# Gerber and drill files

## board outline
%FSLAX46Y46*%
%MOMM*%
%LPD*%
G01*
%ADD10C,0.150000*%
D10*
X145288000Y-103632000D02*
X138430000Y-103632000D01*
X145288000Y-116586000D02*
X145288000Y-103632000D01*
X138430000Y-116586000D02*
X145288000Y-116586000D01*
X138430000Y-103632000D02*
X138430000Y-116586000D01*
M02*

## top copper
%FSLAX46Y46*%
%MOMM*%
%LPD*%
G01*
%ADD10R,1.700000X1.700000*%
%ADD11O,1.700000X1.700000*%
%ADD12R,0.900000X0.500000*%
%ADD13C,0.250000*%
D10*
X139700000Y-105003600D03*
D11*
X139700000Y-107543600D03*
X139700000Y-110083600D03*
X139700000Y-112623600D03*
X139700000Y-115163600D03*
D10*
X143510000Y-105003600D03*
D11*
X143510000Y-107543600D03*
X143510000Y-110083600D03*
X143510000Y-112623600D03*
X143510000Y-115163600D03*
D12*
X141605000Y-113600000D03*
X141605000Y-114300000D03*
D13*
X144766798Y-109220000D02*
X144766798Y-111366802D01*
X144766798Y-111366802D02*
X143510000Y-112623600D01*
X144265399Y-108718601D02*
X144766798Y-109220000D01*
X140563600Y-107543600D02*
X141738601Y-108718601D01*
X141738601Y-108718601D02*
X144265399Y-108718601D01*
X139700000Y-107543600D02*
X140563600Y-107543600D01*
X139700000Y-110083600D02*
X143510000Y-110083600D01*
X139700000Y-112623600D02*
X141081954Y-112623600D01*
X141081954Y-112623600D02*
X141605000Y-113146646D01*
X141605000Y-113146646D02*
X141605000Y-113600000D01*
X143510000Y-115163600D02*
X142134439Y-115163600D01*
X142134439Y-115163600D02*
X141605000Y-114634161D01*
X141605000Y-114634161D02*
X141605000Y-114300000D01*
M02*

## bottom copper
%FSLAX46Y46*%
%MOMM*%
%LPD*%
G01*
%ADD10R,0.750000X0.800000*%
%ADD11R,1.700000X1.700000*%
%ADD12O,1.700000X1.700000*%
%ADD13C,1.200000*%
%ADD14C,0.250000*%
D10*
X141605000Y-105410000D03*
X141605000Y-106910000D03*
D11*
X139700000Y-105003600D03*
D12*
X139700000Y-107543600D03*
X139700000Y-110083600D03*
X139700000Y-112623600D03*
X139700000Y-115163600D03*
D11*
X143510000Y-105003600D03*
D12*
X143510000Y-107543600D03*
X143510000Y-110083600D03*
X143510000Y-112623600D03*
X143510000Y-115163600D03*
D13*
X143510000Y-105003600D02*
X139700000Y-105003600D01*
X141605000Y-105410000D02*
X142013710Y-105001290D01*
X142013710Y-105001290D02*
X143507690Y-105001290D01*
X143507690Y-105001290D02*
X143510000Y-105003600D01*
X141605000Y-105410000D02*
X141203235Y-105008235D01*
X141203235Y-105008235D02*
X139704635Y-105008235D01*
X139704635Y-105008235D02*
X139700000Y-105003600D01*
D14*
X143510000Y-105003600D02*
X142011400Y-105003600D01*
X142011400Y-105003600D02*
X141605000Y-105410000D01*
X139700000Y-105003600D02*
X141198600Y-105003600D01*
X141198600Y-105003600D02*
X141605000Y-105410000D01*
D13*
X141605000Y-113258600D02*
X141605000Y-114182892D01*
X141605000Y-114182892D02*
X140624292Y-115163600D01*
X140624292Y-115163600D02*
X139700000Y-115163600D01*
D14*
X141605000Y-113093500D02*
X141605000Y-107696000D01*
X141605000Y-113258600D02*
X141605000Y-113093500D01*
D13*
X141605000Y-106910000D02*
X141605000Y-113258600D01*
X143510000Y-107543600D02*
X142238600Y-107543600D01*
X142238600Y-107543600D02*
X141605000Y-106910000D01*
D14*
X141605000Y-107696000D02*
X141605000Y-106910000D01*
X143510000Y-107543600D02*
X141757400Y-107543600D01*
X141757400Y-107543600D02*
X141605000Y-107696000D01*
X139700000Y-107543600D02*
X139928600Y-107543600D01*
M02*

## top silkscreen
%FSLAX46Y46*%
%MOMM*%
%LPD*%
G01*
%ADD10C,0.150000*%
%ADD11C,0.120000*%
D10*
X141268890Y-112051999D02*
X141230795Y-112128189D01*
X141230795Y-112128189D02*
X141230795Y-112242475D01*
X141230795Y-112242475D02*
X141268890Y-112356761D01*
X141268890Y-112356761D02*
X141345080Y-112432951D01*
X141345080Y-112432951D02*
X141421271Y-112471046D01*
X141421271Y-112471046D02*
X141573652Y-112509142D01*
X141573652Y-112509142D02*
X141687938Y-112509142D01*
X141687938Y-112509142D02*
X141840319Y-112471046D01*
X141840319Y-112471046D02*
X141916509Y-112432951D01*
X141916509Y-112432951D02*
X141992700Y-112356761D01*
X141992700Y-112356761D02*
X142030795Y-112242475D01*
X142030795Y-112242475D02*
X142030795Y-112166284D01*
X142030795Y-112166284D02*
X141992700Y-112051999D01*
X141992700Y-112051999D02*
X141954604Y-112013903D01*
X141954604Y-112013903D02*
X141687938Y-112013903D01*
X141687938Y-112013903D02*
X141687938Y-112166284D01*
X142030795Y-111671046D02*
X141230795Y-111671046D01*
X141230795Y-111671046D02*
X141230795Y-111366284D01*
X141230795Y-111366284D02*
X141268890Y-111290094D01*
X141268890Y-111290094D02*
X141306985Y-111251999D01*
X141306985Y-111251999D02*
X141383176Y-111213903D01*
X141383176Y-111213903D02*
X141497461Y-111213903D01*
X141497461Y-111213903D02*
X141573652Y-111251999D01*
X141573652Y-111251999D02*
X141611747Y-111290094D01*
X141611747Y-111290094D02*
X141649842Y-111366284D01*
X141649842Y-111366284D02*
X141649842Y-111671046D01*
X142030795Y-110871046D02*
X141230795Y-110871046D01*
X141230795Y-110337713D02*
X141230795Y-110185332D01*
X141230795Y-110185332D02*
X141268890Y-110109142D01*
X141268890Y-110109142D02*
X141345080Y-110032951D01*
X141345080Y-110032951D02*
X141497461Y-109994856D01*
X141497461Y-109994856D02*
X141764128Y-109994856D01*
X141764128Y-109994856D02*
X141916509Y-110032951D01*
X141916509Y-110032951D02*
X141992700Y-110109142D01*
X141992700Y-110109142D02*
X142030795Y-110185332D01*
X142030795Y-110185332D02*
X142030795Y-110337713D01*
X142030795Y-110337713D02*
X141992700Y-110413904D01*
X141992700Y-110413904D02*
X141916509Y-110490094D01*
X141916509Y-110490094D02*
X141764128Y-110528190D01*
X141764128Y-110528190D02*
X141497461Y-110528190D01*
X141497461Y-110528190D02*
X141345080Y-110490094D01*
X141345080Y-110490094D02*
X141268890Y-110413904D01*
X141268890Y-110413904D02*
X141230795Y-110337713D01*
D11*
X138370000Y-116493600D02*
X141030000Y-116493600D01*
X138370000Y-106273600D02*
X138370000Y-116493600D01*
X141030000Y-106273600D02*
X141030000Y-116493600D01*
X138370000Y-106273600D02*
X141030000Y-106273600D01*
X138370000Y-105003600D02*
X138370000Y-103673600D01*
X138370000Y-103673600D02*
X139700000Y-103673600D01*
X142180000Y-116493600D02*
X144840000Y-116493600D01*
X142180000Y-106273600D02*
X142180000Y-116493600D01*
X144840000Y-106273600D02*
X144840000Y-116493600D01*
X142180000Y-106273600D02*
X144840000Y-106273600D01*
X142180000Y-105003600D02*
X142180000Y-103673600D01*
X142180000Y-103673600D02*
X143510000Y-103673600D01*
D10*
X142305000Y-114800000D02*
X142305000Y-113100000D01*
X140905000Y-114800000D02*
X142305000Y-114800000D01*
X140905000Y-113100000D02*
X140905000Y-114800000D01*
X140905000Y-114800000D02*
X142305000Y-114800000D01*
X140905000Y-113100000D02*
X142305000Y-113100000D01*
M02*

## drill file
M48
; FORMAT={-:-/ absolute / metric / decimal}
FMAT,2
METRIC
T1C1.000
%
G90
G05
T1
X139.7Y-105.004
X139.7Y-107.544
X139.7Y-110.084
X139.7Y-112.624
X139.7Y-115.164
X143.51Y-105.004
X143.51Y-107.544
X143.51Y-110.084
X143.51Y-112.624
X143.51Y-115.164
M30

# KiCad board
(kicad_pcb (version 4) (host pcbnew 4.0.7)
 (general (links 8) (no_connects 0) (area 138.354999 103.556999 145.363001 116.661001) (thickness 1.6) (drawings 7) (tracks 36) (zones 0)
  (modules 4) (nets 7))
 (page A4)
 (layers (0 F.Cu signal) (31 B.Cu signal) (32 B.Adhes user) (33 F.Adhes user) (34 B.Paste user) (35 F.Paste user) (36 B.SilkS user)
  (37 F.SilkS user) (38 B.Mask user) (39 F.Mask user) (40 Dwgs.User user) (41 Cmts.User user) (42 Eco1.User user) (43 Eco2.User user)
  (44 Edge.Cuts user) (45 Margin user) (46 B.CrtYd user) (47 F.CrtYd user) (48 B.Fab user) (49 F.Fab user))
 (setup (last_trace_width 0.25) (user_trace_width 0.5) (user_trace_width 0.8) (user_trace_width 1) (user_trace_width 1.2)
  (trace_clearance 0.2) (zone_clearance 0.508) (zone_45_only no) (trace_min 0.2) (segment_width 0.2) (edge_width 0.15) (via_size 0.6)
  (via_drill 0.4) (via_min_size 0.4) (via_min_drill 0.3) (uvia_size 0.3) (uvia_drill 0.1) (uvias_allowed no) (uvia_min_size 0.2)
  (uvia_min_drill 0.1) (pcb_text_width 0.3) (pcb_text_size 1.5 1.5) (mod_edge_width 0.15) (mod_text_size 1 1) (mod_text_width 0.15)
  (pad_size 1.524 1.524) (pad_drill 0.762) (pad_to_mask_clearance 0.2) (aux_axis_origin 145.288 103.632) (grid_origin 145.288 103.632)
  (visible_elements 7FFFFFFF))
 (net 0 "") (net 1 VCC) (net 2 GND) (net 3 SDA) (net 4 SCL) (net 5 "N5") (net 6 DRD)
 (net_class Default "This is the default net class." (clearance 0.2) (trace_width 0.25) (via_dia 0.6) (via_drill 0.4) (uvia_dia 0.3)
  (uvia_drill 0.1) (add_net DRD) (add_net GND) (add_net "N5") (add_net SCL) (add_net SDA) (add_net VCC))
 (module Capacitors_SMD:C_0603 (layer B.Cu) (at 141.605 106.16 90)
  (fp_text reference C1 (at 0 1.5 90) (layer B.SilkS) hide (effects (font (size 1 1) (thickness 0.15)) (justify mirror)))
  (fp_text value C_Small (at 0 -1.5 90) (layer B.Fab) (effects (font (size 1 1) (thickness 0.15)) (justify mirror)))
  (pad 2 smd rect (at 0.75 0 90) (size 0.8 0.75) (layers B.Cu B.Paste B.Mask) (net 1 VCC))
  (pad 1 smd rect (at -0.75 0 90) (size 0.8 0.75) (layers B.Cu B.Paste B.Mask) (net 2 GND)))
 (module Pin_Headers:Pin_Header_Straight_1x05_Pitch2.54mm (layer F.Cu) (at 139.7 105.0036)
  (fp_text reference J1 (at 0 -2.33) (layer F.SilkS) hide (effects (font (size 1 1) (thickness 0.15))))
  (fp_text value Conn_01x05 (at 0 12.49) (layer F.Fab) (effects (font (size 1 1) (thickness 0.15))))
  (fp_line (start -1.33 11.49) (end 1.33 11.49) (layer F.SilkS) (width 0.12))
  (fp_line (start -1.33 1.27) (end -1.33 11.49) (layer F.SilkS) (width 0.12))
  (fp_line (start 1.33 1.27) (end 1.33 11.49) (layer F.SilkS) (width 0.12))
  (fp_line (start -1.33 1.27) (end 1.33 1.27) (layer F.SilkS) (width 0.12))
  (fp_line (start -1.33 0) (end -1.33 -1.33) (layer F.SilkS) (width 0.12))
  (fp_line (start -1.33 -1.33) (end 0 -1.33) (layer F.SilkS) (width 0.12))
  (pad 1 thru_hole rect (at 0 0) (size 1.7 1.7) (drill 1) (layers *.Cu *.Mask) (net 1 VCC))
  (pad 2 thru_hole oval (at 0 2.54) (size 1.7 1.7) (drill 1) (layers *.Cu *.Mask) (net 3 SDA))
  (pad 3 thru_hole oval (at 0 5.08) (size 1.7 1.7) (drill 1) (layers *.Cu *.Mask) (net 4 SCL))
  (pad 4 thru_hole oval (at 0 7.62) (size 1.7 1.7) (drill 1) (layers *.Cu *.Mask) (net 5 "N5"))
  (pad 5 thru_hole oval (at 0 10.16) (size 1.7 1.7) (drill 1) (layers *.Cu *.Mask) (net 2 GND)))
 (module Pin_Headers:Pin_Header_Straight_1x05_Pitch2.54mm (layer F.Cu) (at 143.51 105.0036)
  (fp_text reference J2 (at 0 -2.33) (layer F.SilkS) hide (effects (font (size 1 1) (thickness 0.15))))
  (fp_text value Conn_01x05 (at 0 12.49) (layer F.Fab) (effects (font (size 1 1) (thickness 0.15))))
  (fp_line (start -1.33 11.49) (end 1.33 11.49) (layer F.SilkS) (width 0.12))
  (fp_line (start -1.33 1.27) (end -1.33 11.49) (layer F.SilkS) (width 0.12))
  (fp_line (start 1.33 1.27) (end 1.33 11.49) (layer F.SilkS) (width 0.12))
  (fp_line (start -1.33 1.27) (end 1.33 1.27) (layer F.SilkS) (width 0.12))
  (fp_line (start -1.33 0) (end -1.33 -1.33) (layer F.SilkS) (width 0.12))
  (fp_line (start -1.33 -1.33) (end 0 -1.33) (layer F.SilkS) (width 0.12))
  (pad 1 thru_hole rect (at 0 0) (size 1.7 1.7) (drill 1) (layers *.Cu *.Mask) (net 1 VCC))
  (pad 2 thru_hole oval (at 0 2.54) (size 1.7 1.7) (drill 1) (layers *.Cu *.Mask) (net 2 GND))
  (pad 3 thru_hole oval (at 0 5.08) (size 1.7 1.7) (drill 1) (layers *.Cu *.Mask) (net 4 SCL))
  (pad 4 thru_hole oval (at 0 7.62) (size 1.7 1.7) (drill 1) (layers *.Cu *.Mask) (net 3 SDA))
  (pad 5 thru_hole oval (at 0 10.16) (size 1.7 1.7) (drill 1) (layers *.Cu *.Mask) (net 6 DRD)))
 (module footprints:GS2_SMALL (layer F.Cu) (at 141.605 114.3)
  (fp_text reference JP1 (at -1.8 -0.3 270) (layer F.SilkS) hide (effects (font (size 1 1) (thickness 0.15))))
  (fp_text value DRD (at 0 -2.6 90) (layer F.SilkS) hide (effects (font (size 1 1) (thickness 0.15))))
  (fp_line (start 0.7 0.5) (end 0.7 -1.2) (layer F.SilkS) (width 0.15))
  (fp_line (start -0.7 0.5) (end 0.7 0.5) (layer F.SilkS) (width 0.15))
  (fp_line (start -0.7 -1.2) (end -0.7 0.5) (layer F.SilkS) (width 0.15))
  (fp_line (start -0.7 0.5) (end 0.7 0.5) (layer F.SilkS) (width 0.15))
  (fp_line (start -0.7 -1.2) (end 0.7 -1.2) (layer F.SilkS) (width 0.15))
  (pad 1 smd rect (at 0 -0.7) (size 0.9 0.5) (layers F.Cu F.Paste F.Mask) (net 5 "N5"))
  (pad 2 smd rect (at 0 0) (size 0.9 0.5) (layers F.Cu F.Paste F.Mask) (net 6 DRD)))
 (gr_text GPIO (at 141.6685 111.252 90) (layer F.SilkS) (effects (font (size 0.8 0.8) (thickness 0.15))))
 (gr_line (start 145.288 103.632) (end 138.43 103.632) (layer Edge.Cuts) (width 0.15))
 (gr_line (start 145.288 116.586) (end 145.288 103.632) (layer Edge.Cuts) (width 0.15))
 (gr_line (start 138.43 116.586) (end 145.288 116.586) (layer Edge.Cuts) (width 0.15))
 (gr_line (start 138.43 103.632) (end 138.43 116.586) (layer Edge.Cuts) (width 0.15))
 (segment (start 143.51 105.0036) (end 139.7 105.0036) (width 1.2) (layer B.Cu) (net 1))
 (segment (start 141.605 105.41) (end 142.01371 105.00129) (width 1.2) (layer B.Cu) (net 1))
 (segment (start 142.01371 105.00129) (end 143.50769 105.00129) (width 1.2) (layer B.Cu) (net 1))
 (segment (start 143.50769 105.00129) (end 143.51 105.0036) (width 1.2) (layer B.Cu) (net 1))
 (segment (start 141.605 105.41) (end 141.203235 105.008235) (width 1.2) (layer B.Cu) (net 1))
 (segment (start 141.203235 105.008235) (end 139.704635 105.008235) (width 1.2) (layer B.Cu) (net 1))
 (segment (start 139.704635 105.008235) (end 139.7 105.0036) (width 1.2) (layer B.Cu) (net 1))
 (segment (start 143.51 105.0036) (end 142.0114 105.0036) (width 0.25) (layer B.Cu) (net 1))
 (segment (start 142.0114 105.0036) (end 141.605 105.41) (width 0.25) (layer B.Cu) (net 1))
 (segment (start 139.7 105.0036) (end 141.1986 105.0036) (width 0.25) (layer B.Cu) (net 1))
 (segment (start 141.1986 105.0036) (end 141.605 105.41) (width 0.25) (layer B.Cu) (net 1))
 (segment (start 141.605 113.2586) (end 141.605 114.182892) (width 1.2) (layer B.Cu) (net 2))
 (segment (start 141.605 114.182892) (end 140.624292 115.1636) (width 1.2) (layer B.Cu) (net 2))
 (segment (start 140.624292 115.1636) (end 139.7 115.1636) (width 1.2) (layer B.Cu) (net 2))
 (segment (start 141.605 113.0935) (end 141.605 107.696) (width 0.25) (layer B.Cu) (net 2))
 (segment (start 141.605 113.2586) (end 141.605 113.0935) (width 0.25) (layer B.Cu) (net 2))
 (segment (start 141.605 106.91) (end 141.605 113.2586) (width 1.2) (layer B.Cu) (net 2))
 (segment (start 143.51 107.5436) (end 142.2386 107.5436) (width 1.2) (layer B.Cu) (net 2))
 (segment (start 142.2386 107.5436) (end 141.605 106.91) (width 1.2) (layer B.Cu) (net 2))
 (segment (start 141.605 107.696) (end 141.605 106.91) (width 0.25) (layer B.Cu) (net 2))
 (segment (start 143.51 107.5436) (end 141.7574 107.5436) (width 0.25) (layer B.Cu) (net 2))
 (segment (start 141.7574 107.5436) (end 141.605 107.696) (width 0.25) (layer B.Cu) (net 2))
 (segment (start 144.766798 109.22) (end 144.766798 111.366802) (width 0.25) (layer F.Cu) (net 3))
 (segment (start 144.766798 111.366802) (end 143.51 112.6236) (width 0.25) (layer F.Cu) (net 3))
 (segment (start 144.265399 108.718601) (end 144.766798 109.22) (width 0.25) (layer F.Cu) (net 3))
 (segment (start 140.5636 107.5436) (end 141.738601 108.718601) (width 0.25) (layer F.Cu) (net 3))
 (segment (start 141.738601 108.718601) (end 144.265399 108.718601) (width 0.25) (layer F.Cu) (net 3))
 (segment (start 139.7 107.5436) (end 140.5636 107.5436) (width 0.25) (layer F.Cu) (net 3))
 (segment (start 139.7 107.5436) (end 139.9286 107.5436) (width 0.25) (layer B.Cu) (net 3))
 (segment (start 139.7 110.0836) (end 143.51 110.0836) (width 0.25) (layer F.Cu) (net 4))
 (segment (start 139.7 112.6236) (end 141.081954 112.6236) (width 0.25) (layer F.Cu) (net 5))
 (segment (start 141.081954 112.6236) (end 141.605 113.146646) (width 0.25) (layer F.Cu) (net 5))
 (segment (start 141.605 113.146646) (end 141.605 113.6) (width 0.25) (layer F.Cu) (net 5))
 (segment (start 143.51 115.1636) (end 142.134439 115.1636) (width 0.25) (layer F.Cu) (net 6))
 (segment (start 142.134439 115.1636) (end 141.605 114.634161) (width 0.25) (layer F.Cu) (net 6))
 (segment (start 141.605 114.634161) (end 141.605 114.3) (width 0.25) (layer F.Cu) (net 6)))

